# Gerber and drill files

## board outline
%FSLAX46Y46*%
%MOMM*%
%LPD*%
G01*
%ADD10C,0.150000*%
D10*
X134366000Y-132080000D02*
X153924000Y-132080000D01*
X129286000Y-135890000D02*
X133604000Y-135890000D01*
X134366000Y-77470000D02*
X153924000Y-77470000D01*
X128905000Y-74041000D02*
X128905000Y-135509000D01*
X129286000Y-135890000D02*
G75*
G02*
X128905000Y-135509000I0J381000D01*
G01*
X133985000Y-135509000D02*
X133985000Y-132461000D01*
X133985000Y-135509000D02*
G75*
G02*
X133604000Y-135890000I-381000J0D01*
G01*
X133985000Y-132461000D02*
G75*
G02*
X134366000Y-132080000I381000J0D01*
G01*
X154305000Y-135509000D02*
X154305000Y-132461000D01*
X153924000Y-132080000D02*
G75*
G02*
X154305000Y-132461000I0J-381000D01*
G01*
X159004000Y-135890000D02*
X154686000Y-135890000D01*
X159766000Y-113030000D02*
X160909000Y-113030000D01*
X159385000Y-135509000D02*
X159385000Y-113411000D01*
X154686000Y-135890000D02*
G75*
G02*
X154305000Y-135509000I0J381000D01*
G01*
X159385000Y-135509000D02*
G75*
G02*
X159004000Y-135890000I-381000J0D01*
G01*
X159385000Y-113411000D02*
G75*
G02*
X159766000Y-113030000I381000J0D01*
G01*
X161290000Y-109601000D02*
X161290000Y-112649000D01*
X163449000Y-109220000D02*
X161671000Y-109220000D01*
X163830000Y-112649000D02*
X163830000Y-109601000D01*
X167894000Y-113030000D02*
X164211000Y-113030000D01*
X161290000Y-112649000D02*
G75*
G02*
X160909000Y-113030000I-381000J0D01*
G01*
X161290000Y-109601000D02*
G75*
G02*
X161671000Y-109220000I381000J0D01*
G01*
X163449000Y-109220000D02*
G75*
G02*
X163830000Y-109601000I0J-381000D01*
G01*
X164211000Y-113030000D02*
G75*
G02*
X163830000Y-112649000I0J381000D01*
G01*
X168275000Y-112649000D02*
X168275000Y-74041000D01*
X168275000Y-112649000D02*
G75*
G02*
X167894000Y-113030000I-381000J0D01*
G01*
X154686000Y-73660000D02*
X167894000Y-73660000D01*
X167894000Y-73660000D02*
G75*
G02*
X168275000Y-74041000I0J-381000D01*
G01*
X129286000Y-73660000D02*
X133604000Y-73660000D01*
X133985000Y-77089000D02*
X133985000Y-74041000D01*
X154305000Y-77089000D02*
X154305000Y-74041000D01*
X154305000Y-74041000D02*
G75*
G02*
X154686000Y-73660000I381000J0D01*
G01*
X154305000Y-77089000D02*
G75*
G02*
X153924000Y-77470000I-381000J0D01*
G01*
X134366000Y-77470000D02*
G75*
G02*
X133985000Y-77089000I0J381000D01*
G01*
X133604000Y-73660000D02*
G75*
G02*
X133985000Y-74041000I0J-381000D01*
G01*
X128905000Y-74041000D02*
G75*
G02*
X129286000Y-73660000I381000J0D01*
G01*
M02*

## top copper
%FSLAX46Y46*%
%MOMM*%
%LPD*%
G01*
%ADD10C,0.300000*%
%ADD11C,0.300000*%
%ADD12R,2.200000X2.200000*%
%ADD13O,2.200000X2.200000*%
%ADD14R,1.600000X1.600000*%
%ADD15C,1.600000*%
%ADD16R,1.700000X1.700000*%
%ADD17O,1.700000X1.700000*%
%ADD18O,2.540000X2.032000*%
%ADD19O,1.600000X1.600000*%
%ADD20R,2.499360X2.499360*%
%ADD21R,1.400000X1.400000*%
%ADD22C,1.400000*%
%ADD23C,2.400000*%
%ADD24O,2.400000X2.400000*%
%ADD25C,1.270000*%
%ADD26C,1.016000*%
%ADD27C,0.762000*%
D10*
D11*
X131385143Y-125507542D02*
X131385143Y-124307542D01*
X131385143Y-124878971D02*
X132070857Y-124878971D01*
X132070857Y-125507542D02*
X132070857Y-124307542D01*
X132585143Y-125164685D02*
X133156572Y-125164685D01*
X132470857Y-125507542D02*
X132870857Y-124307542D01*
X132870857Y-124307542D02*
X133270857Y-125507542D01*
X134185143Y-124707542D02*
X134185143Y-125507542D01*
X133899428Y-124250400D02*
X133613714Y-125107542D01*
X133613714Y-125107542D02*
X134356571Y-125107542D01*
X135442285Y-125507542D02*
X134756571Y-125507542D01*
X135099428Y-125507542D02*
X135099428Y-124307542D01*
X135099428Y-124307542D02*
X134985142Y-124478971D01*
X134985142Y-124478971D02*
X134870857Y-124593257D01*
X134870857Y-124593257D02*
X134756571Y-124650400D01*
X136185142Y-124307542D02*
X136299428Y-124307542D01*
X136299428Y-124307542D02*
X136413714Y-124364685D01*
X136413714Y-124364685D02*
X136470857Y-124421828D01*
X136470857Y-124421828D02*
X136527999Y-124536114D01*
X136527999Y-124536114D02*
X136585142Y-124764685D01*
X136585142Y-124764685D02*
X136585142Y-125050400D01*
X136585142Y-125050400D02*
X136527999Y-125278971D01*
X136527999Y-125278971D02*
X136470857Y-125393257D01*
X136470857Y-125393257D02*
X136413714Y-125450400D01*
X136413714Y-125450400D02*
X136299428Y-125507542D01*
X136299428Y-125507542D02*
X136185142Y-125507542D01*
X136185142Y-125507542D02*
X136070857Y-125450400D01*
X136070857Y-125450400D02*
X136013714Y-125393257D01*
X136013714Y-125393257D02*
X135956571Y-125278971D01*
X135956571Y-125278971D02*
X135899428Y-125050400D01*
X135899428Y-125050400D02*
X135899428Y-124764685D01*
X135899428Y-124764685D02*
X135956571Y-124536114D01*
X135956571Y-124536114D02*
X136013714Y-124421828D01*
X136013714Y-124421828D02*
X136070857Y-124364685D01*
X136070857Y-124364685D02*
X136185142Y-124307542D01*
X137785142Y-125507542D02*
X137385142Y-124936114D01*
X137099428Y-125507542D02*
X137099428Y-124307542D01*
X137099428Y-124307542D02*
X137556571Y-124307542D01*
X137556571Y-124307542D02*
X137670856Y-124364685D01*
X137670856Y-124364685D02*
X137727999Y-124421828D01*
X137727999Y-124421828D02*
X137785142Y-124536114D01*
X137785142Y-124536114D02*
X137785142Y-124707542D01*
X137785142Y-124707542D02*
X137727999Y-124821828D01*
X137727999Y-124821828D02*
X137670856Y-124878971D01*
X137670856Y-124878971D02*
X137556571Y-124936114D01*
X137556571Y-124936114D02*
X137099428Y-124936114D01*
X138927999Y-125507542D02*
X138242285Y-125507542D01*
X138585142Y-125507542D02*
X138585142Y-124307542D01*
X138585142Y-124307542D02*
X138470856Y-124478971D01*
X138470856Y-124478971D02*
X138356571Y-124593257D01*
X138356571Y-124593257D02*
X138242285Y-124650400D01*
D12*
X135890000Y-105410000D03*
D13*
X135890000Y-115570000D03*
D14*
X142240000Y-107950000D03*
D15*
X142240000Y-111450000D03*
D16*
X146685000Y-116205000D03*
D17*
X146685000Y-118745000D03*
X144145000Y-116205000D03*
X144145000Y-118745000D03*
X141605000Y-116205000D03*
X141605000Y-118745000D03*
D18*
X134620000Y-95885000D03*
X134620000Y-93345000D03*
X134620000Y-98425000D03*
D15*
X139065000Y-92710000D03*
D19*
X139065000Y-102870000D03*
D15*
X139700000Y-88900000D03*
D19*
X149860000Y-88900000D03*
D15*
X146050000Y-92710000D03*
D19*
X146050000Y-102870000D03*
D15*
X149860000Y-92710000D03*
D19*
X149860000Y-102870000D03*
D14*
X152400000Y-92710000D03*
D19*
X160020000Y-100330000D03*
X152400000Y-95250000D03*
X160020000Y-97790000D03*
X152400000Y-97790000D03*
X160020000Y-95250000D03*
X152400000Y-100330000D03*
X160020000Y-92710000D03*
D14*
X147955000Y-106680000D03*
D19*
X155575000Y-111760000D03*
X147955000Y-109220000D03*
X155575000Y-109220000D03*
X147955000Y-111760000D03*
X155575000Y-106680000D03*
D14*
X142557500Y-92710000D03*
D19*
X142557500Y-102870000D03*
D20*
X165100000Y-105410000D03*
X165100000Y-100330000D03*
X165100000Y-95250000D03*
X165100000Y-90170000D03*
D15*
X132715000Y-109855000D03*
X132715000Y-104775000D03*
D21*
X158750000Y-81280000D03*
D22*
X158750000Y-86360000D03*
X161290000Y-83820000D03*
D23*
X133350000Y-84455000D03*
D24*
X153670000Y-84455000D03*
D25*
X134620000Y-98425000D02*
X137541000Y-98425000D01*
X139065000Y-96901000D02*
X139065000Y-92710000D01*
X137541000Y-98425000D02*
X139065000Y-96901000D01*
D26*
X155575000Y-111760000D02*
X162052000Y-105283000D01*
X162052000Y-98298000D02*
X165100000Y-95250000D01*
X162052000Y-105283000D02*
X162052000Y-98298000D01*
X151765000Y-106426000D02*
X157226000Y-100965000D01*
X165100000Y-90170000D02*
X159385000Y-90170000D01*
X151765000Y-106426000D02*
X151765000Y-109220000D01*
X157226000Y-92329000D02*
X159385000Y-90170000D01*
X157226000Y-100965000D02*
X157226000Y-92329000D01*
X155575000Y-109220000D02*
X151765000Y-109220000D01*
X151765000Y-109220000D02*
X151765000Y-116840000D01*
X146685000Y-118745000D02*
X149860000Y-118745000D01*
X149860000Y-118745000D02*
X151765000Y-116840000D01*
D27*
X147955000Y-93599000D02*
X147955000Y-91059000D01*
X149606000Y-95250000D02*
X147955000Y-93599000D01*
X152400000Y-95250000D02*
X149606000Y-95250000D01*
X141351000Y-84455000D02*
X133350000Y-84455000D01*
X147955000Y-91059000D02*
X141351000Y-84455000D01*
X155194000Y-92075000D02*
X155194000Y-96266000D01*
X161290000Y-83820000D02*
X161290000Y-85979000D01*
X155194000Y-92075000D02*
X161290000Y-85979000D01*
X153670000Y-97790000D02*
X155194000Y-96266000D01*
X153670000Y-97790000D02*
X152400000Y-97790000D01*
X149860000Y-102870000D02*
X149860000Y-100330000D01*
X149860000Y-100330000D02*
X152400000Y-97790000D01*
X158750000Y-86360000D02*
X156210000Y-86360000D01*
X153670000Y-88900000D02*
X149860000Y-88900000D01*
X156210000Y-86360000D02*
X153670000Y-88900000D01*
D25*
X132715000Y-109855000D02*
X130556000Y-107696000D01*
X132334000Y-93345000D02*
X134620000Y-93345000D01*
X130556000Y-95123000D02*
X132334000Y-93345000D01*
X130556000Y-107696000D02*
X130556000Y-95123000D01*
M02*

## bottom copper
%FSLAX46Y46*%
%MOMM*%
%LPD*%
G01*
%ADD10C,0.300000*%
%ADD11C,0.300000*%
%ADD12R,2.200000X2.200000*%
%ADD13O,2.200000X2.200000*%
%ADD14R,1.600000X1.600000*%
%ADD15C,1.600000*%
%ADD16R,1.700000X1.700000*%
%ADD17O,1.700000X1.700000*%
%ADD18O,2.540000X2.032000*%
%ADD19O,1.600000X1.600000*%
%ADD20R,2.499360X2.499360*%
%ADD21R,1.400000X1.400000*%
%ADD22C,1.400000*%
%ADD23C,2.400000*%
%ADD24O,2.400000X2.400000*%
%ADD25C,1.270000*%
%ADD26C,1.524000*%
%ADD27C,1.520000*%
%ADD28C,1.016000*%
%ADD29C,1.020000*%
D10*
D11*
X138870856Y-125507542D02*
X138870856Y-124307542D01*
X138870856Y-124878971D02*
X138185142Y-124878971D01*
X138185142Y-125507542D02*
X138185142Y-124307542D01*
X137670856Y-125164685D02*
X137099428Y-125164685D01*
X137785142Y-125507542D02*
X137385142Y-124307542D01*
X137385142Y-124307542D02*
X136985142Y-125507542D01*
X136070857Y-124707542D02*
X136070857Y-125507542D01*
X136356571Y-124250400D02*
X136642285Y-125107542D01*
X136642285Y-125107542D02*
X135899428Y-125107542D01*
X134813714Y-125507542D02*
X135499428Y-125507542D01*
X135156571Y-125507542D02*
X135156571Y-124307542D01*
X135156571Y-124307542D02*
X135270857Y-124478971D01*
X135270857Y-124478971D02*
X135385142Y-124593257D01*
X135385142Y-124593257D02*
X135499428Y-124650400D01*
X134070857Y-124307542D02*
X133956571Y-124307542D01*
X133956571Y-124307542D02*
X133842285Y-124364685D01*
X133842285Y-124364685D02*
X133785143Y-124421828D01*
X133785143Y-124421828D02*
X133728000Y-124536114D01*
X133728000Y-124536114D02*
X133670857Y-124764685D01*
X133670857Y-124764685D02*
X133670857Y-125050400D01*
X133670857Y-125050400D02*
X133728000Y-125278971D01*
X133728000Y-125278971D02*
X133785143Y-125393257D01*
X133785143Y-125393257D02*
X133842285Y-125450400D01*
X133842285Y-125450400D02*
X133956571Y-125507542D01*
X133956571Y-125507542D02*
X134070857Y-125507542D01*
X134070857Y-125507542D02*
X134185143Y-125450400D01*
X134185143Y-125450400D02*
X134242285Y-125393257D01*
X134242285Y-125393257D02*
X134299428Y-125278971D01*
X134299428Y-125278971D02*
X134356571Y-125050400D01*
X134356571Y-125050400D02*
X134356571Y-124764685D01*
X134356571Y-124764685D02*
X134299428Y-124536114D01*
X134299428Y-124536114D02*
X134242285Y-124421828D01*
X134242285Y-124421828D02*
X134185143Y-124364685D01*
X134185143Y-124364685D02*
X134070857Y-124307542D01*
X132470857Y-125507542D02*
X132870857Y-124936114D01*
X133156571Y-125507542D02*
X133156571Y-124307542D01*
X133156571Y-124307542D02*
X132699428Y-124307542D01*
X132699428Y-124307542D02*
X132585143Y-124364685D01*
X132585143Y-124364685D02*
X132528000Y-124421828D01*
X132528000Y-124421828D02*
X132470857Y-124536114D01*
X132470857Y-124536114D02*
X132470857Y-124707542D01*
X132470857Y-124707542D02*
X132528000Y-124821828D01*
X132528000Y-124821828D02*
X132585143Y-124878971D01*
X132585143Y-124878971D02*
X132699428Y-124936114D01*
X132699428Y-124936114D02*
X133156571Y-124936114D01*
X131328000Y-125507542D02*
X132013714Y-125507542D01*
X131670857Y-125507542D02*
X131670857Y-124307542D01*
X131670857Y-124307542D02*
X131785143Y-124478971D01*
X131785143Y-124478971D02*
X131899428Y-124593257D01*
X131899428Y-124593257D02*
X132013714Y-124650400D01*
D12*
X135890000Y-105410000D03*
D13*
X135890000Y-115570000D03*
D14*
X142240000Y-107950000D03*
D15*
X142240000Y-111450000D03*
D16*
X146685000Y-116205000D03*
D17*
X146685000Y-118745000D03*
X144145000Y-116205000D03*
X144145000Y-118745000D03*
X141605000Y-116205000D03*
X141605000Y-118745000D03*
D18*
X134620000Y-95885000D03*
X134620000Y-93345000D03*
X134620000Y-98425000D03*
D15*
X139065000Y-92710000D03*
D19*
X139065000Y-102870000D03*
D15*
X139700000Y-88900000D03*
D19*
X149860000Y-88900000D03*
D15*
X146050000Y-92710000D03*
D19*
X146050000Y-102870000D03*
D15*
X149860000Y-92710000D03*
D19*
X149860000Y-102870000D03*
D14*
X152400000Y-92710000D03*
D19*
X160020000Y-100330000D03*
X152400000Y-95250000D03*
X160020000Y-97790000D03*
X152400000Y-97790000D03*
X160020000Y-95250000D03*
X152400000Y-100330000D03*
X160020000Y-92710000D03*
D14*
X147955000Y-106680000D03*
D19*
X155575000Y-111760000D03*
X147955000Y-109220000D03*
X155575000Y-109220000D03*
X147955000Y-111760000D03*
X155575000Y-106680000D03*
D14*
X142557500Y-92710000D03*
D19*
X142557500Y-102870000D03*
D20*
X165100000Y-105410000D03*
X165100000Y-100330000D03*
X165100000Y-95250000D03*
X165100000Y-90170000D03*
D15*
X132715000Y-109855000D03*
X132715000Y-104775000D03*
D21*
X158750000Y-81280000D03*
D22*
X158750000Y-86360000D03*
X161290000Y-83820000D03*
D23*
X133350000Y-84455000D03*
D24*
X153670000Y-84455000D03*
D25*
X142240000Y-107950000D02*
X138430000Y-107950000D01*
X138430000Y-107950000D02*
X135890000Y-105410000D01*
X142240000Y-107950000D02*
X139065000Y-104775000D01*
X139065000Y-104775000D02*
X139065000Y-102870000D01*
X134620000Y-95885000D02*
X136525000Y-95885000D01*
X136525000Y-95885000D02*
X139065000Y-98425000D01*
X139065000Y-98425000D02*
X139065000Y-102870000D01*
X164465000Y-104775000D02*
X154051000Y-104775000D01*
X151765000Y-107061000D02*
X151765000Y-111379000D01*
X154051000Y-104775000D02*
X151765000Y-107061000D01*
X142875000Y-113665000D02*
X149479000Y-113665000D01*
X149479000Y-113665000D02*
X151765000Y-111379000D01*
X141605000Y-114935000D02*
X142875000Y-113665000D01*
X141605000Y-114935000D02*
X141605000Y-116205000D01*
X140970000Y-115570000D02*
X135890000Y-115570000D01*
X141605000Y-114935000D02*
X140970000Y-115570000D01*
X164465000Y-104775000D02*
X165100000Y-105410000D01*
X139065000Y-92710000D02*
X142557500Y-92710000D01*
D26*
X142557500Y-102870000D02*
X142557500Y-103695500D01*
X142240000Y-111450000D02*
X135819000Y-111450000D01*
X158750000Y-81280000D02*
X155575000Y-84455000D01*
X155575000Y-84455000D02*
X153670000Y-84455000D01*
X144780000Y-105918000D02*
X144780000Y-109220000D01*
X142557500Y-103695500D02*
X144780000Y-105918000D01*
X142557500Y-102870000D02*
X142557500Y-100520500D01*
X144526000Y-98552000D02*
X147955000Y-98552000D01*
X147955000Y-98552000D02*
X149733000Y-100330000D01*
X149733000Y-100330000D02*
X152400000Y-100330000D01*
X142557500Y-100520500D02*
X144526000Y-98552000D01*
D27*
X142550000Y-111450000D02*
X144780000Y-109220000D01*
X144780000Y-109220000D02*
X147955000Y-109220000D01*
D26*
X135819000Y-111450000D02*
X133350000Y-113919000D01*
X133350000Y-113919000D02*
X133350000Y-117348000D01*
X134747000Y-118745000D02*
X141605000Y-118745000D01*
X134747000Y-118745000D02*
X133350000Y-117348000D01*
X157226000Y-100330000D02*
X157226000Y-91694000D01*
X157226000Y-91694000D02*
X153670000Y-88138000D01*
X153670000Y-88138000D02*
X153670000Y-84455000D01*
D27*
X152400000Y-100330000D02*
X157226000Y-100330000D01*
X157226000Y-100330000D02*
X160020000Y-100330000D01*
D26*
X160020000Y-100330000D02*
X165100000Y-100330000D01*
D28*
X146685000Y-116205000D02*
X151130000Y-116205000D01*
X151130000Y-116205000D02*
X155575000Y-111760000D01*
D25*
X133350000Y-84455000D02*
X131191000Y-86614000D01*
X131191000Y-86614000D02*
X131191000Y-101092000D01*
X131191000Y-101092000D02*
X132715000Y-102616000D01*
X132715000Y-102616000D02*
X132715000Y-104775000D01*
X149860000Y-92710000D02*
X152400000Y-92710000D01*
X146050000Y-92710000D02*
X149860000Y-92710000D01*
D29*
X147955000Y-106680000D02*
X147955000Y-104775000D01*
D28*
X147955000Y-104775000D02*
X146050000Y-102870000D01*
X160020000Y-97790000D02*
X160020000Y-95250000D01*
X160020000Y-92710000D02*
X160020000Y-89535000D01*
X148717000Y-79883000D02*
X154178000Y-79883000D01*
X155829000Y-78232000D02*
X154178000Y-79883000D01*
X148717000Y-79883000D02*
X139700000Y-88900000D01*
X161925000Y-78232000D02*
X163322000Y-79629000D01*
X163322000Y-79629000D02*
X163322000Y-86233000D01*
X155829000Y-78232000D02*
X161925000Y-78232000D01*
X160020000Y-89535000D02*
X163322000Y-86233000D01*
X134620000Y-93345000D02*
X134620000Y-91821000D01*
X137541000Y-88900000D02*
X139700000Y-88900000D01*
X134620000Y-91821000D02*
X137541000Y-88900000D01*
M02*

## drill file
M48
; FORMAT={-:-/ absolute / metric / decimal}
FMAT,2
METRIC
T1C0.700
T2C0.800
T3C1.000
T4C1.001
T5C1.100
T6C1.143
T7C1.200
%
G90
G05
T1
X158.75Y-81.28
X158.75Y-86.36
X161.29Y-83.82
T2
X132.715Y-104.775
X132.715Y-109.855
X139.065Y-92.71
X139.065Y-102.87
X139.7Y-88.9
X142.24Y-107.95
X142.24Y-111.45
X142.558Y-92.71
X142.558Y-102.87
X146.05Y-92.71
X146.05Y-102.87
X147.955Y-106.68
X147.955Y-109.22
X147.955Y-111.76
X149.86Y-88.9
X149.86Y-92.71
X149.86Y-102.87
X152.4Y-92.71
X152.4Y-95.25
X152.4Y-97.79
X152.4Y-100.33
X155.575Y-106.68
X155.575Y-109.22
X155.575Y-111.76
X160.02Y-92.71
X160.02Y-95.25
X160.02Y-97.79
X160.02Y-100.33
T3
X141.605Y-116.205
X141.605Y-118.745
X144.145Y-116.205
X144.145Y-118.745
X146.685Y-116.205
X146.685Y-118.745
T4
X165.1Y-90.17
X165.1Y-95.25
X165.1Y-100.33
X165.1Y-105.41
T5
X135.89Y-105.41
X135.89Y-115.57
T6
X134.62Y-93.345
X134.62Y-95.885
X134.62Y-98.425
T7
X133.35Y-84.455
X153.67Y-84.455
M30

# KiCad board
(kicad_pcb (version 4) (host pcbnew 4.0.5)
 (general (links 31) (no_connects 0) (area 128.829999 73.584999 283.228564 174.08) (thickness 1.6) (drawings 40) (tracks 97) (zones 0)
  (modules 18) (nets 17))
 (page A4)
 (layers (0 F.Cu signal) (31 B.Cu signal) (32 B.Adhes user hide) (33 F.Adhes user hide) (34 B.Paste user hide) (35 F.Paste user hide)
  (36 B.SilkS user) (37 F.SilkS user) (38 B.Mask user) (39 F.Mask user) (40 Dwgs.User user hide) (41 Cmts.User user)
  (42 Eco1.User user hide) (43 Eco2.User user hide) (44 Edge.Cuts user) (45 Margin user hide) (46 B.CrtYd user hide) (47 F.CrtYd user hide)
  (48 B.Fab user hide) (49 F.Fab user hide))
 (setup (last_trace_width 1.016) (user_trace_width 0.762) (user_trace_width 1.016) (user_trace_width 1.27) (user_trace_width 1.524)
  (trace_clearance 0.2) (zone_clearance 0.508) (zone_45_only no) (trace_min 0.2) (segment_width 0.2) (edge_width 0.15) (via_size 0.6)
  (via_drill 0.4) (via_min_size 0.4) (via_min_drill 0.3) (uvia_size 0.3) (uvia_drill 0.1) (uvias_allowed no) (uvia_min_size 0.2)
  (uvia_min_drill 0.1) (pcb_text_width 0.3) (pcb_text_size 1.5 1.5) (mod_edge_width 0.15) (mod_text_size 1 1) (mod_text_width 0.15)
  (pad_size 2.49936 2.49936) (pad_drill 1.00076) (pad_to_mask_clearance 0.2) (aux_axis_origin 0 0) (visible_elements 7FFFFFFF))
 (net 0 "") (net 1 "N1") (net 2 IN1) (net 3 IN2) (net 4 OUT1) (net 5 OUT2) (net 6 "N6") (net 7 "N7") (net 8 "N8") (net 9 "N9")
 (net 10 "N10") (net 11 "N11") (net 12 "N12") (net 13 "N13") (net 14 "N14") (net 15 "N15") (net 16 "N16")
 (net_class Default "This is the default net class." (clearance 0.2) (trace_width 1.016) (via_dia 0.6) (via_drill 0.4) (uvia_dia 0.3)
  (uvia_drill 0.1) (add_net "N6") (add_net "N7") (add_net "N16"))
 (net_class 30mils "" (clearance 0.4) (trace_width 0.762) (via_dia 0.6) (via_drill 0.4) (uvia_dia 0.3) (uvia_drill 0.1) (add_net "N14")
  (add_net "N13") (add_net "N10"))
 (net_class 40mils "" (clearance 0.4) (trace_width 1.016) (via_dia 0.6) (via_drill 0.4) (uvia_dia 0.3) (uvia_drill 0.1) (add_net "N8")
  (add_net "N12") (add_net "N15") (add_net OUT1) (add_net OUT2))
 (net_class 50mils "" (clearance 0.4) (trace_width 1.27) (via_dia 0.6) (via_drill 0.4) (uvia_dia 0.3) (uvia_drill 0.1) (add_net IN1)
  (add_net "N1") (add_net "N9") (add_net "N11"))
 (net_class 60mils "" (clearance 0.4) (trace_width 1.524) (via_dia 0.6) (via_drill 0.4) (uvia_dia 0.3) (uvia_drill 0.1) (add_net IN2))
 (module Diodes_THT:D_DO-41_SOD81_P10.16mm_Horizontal (layer F.Cu) (at 135.89 105.41 270)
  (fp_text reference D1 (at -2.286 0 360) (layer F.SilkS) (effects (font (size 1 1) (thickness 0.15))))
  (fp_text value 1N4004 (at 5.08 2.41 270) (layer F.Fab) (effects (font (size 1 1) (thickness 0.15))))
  (pad 1 thru_hole rect (at 0 0 270) (size 2.2 2.2) (drill 1.1) (layers *.Cu *.Mask) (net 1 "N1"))
  (pad 2 thru_hole oval (at 10.16 0 270) (size 2.2 2.2) (drill 1.1) (layers *.Cu *.Mask) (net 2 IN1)))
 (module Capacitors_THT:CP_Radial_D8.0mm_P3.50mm (layer F.Cu) (at 142.24 107.95 270)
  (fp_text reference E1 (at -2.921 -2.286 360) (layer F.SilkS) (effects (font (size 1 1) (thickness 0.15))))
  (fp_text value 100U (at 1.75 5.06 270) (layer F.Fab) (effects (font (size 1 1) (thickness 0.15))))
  (pad 1 thru_hole rect (at 0 0 270) (size 1.6 1.6) (drill 0.8) (layers *.Cu *.Mask) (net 1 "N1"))
  (pad 2 thru_hole circle (at 3.5 0 270) (size 1.6 1.6) (drill 0.8) (layers *.Cu *.Mask) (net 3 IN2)))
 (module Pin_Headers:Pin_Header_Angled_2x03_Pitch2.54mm (layer F.Cu) (at 146.685 116.205 270)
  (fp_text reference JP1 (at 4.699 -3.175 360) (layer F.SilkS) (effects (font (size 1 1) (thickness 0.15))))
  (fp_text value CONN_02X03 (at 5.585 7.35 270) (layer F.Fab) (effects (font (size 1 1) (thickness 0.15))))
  (pad 1 thru_hole rect (at 0 0 270) (size 1.7 1.7) (drill 1) (layers *.Cu *.Mask) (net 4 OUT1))
  (pad 2 thru_hole oval (at 2.54 0 270) (size 1.7 1.7) (drill 1) (layers *.Cu *.Mask) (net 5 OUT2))
  (pad 3 thru_hole oval (at 0 2.54 270) (size 1.7 1.7) (drill 1) (layers *.Cu *.Mask) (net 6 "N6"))
  (pad 4 thru_hole oval (at 2.54 2.54 270) (size 1.7 1.7) (drill 1) (layers *.Cu *.Mask) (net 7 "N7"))
  (pad 5 thru_hole oval (at 0 5.08 270) (size 1.7 1.7) (drill 1) (layers *.Cu *.Mask) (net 2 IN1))
  (pad 6 thru_hole oval (at 2.54 5.08 270) (size 1.7 1.7) (drill 1) (layers *.Cu *.Mask) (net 3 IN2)))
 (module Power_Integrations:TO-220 (layer F.Cu) (at 134.62 95.885 90)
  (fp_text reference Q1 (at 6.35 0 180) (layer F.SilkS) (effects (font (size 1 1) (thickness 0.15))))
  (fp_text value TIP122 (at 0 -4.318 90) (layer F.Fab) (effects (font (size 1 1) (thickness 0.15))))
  (pad 2 thru_hole oval (at 0 0 90) (size 2.032 2.54) (drill 1.143) (layers *.Cu *.Mask) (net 1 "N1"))
  (pad 3 thru_hole oval (at 2.54 0 90) (size 2.032 2.54) (drill 1.143) (layers *.Cu *.Mask) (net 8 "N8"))
  (pad 1 thru_hole oval (at -2.54 0 90) (size 2.032 2.54) (drill 1.143) (layers *.Cu *.Mask) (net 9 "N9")))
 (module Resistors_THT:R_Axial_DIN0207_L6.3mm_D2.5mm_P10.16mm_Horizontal (layer F.Cu) (at 139.065 92.71 270)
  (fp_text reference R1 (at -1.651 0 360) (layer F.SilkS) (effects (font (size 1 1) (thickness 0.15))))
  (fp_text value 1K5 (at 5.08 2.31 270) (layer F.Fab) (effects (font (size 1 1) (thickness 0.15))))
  (pad 1 thru_hole circle (at 0 0 270) (size 1.6 1.6) (drill 0.8) (layers *.Cu *.Mask) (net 9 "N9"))
  (pad 2 thru_hole oval (at 10.16 0 270) (size 1.6 1.6) (drill 0.8) (layers *.Cu *.Mask) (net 1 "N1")))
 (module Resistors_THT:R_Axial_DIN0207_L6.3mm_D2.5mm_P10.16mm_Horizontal (layer F.Cu) (at 139.7 88.9)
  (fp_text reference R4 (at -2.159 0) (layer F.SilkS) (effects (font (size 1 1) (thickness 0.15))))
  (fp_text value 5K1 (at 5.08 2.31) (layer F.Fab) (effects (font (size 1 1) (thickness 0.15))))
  (pad 1 thru_hole circle (at 0 0) (size 1.6 1.6) (drill 0.8) (layers *.Cu *.Mask) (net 8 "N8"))
  (pad 2 thru_hole oval (at 10.16 0) (size 1.6 1.6) (drill 0.8) (layers *.Cu *.Mask) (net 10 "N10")))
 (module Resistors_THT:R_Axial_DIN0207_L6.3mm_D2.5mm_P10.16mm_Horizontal (layer F.Cu) (at 146.05 92.71 270)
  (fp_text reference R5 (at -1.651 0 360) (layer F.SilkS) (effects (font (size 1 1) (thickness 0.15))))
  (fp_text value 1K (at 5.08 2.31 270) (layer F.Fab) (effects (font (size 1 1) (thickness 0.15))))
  (pad 1 thru_hole circle (at 0 0 270) (size 1.6 1.6) (drill 0.8) (layers *.Cu *.Mask) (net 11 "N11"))
  (pad 2 thru_hole oval (at 10.16 0 270) (size 1.6 1.6) (drill 0.8) (layers *.Cu *.Mask) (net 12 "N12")))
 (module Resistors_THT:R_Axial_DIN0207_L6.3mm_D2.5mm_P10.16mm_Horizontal (layer F.Cu) (at 149.86 92.71 270)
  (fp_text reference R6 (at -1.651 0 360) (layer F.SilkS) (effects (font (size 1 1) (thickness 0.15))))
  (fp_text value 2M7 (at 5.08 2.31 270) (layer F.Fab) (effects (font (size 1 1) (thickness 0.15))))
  (pad 1 thru_hole circle (at 0 0 270) (size 1.6 1.6) (drill 0.8) (layers *.Cu *.Mask) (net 11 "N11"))
  (pad 2 thru_hole oval (at 10.16 0 270) (size 1.6 1.6) (drill 0.8) (layers *.Cu *.Mask) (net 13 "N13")))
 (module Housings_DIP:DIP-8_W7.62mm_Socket (layer F.Cu) (at 152.4 92.71)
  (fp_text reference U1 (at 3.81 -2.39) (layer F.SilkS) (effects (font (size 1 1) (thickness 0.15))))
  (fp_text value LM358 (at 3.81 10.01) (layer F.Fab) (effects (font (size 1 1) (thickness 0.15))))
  (pad 1 thru_hole rect (at 0 0) (size 1.6 1.6) (drill 0.8) (layers *.Cu *.Mask) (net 11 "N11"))
  (pad 5 thru_hole oval (at 7.62 7.62) (size 1.6 1.6) (drill 0.8) (layers *.Cu *.Mask) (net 3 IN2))
  (pad 2 thru_hole oval (at 0 2.54) (size 1.6 1.6) (drill 0.8) (layers *.Cu *.Mask) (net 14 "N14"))
  (pad 6 thru_hole oval (at 7.62 5.08) (size 1.6 1.6) (drill 0.8) (layers *.Cu *.Mask) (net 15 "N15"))
  (pad 3 thru_hole oval (at 0 5.08) (size 1.6 1.6) (drill 0.8) (layers *.Cu *.Mask) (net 13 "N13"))
  (pad 7 thru_hole oval (at 7.62 2.54) (size 1.6 1.6) (drill 0.8) (layers *.Cu *.Mask) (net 15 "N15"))
  (pad 4 thru_hole oval (at 0 7.62) (size 1.6 1.6) (drill 0.8) (layers *.Cu *.Mask) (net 3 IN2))
  (pad 8 thru_hole oval (at 7.62 0) (size 1.6 1.6) (drill 0.8) (layers *.Cu *.Mask) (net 8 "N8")))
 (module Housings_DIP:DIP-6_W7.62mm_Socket (layer F.Cu) (at 147.955 106.68)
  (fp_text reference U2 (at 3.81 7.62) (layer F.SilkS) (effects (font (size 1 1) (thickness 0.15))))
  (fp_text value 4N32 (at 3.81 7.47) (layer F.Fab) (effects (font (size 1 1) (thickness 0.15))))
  (pad 1 thru_hole rect (at 0 0) (size 1.6 1.6) (drill 0.8) (layers *.Cu *.Mask) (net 12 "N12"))
  (pad 4 thru_hole oval (at 7.62 5.08) (size 1.6 1.6) (drill 0.8) (layers *.Cu *.Mask) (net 4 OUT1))
  (pad 2 thru_hole oval (at 0 2.54) (size 1.6 1.6) (drill 0.8) (layers *.Cu *.Mask) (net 3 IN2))
  (pad 5 thru_hole oval (at 7.62 2.54) (size 1.6 1.6) (drill 0.8) (layers *.Cu *.Mask) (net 5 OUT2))
  (pad 3 thru_hole oval (at 0 5.08) (size 1.6 1.6) (drill 0.8) (layers *.Cu *.Mask))
  (pad 6 thru_hole oval (at 7.62 0) (size 1.6 1.6) (drill 0.8) (layers *.Cu *.Mask) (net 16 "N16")))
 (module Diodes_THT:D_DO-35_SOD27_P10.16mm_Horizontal (layer F.Cu) (at 142.5575 92.71 270)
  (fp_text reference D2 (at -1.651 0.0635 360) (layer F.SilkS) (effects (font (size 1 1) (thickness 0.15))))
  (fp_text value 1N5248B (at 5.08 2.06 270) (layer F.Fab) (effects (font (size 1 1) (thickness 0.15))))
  (pad 1 thru_hole rect (at 0 0 270) (size 1.6 1.6) (drill 0.8) (layers *.Cu *.Mask) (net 9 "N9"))
  (pad 2 thru_hole oval (at 10.16 0 270) (size 1.6 1.6) (drill 0.8) (layers *.Cu *.Mask) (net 3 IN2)))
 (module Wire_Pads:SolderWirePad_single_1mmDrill (layer F.Cu) (at 165.1 105.41)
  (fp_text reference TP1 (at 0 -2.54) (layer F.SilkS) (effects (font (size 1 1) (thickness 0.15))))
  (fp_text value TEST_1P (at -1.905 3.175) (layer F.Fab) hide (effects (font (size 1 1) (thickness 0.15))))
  (pad 1 thru_hole rect (at 0 0) (size 2.49936 2.49936) (drill 1.00076) (layers *.Cu *.Mask) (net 2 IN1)))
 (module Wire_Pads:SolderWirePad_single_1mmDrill (layer F.Cu) (at 165.1 100.33)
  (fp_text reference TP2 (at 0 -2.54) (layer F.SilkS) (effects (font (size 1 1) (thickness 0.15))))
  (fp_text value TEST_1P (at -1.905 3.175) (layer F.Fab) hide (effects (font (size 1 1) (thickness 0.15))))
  (pad 1 thru_hole rect (at 0 0) (size 2.49936 2.49936) (drill 1.00076) (layers *.Cu *.Mask) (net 3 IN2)))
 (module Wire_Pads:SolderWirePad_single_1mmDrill (layer F.Cu) (at 165.1 95.25)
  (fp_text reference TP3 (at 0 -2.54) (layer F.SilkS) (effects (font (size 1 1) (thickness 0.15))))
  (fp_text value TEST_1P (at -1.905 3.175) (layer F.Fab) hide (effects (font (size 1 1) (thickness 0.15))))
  (pad 1 thru_hole rect (at 0 0) (size 2.49936 2.49936) (drill 1.00076) (layers *.Cu *.Mask) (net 4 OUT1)))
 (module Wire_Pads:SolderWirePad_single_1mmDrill (layer F.Cu) (at 165.1 90.17)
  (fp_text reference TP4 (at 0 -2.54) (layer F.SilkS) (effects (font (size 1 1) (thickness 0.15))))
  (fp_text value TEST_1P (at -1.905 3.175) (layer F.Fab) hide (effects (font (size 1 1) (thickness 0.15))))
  (pad 1 thru_hole rect (at 0 0) (size 2.49936 2.49936) (drill 1.00076) (layers *.Cu *.Mask) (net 5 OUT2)))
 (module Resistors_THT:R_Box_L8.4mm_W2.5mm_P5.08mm (layer F.Cu) (at 132.715 109.855 90)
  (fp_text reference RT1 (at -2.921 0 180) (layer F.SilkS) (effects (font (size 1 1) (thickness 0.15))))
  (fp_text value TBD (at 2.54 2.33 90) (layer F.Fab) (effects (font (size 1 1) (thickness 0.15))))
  (pad 1 thru_hole circle (at 0 0 90) (size 1.6 1.6) (drill 0.8) (layers *.Cu *.Mask) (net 8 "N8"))
  (pad 2 thru_hole circle (at 5.08 0 90) (size 1.6 1.6) (drill 0.8) (layers *.Cu *.Mask) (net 14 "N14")))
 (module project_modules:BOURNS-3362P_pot (layer F.Cu) (at 158.75 83.82 270)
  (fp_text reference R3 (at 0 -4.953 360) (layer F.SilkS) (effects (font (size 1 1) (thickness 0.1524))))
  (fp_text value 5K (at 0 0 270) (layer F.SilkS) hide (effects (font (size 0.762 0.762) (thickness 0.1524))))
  (pad 1 thru_hole rect (at -2.54 0 270) (size 1.4 1.4) (drill 0.7) (layers *.Cu *.Mask F.SilkS) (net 3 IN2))
  (pad 3 thru_hole circle (at 2.54 0 270) (size 1.4 1.4) (drill 0.7) (layers *.Cu *.Mask F.SilkS) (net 10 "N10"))
  (pad 2 thru_hole circle (at 0 -2.54 270) (size 1.4 1.4) (drill 0.7) (layers *.Cu *.Mask F.SilkS) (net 13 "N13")))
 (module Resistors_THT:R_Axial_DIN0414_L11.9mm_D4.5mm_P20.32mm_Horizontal (layer F.Cu) (at 133.35 84.455)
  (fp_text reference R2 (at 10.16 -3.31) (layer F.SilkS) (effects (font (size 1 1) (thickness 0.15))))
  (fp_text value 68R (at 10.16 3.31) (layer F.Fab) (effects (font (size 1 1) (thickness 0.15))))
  (pad 1 thru_hole circle (at 0 0) (size 2.4 2.4) (drill 1.2) (layers *.Cu *.Mask) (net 14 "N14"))
  (pad 2 thru_hole oval (at 20.32 0) (size 2.4 2.4) (drill 1.2) (layers *.Cu *.Mask) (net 3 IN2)))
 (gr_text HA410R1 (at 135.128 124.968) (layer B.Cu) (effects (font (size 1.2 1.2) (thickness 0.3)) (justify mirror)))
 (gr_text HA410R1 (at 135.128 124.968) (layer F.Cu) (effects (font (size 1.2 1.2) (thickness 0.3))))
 (gr_line (start 134.366 132.08) (end 153.924 132.08) (angle 90) (layer Edge.Cuts) (width 0.15))
 (gr_line (start 129.286 135.89) (end 133.604 135.89) (angle 90) (layer Edge.Cuts) (width 0.15))
 (gr_line (start 134.366 77.47) (end 153.924 77.47) (angle 90) (layer Edge.Cuts) (width 0.15))
 (gr_line (start 128.905 74.041) (end 128.905 135.509) (angle 90) (layer Edge.Cuts) (width 0.15))
 (gr_arc (start 129.286 135.509) (end 129.286 135.89) (angle 90) (layer Edge.Cuts) (width 0.15))
 (gr_line (start 133.985 135.509) (end 133.985 132.461) (angle 90) (layer Edge.Cuts) (width 0.15))
 (gr_arc (start 133.604 135.509) (end 133.604 135.89) (angle -90) (layer Edge.Cuts) (width 0.15))
 (gr_arc (start 134.366 132.461) (end 134.366 132.08) (angle -90) (layer Edge.Cuts) (width 0.15))
 (gr_line (start 154.305 135.509) (end 154.305 132.461) (angle 90) (layer Edge.Cuts) (width 0.15))
 (gr_arc (start 153.924 132.461) (end 153.924 132.08) (angle 90) (layer Edge.Cuts) (width 0.15))
 (gr_line (start 159.004 135.89) (end 154.686 135.89) (angle 90) (layer Edge.Cuts) (width 0.15))
 (gr_line (start 159.766 113.03) (end 160.909 113.03) (angle 90) (layer Edge.Cuts) (width 0.15))
 (gr_line (start 159.385 135.509) (end 159.385 113.411) (angle 90) (layer Edge.Cuts) (width 0.15))
 (gr_arc (start 154.686 135.509) (end 154.686 135.89) (angle 90) (layer Edge.Cuts) (width 0.15))
 (gr_arc (start 159.004 135.509) (end 159.004 135.89) (angle -90) (layer Edge.Cuts) (width 0.15))
 (gr_arc (start 159.766 113.411) (end 159.766 113.03) (angle -90) (layer Edge.Cuts) (width 0.15))
 (gr_line (start 161.29 109.601) (end 161.29 112.649) (angle 90) (layer Edge.Cuts) (width 0.15))
 (gr_line (start 163.449 109.22) (end 161.671 109.22) (angle 90) (layer Edge.Cuts) (width 0.15))
 (gr_line (start 163.83 112.649) (end 163.83 109.601) (angle 90) (layer Edge.Cuts) (width 0.15))
 (gr_line (start 167.894 113.03) (end 164.211 113.03) (angle 90) (layer Edge.Cuts) (width 0.15))
 (gr_arc (start 160.909 112.649) (end 160.909 113.03) (angle -90) (layer Edge.Cuts) (width 0.15))
 (gr_arc (start 161.671 109.601) (end 161.671 109.22) (angle -90) (layer Edge.Cuts) (width 0.15))
 (gr_arc (start 163.449 109.601) (end 163.449 109.22) (angle 90) (layer Edge.Cuts) (width 0.15))
 (gr_arc (start 164.211 112.649) (end 164.211 113.03) (angle 90) (layer Edge.Cuts) (width 0.15))
 (gr_line (start 168.275 112.649) (end 168.275 74.041) (angle 90) (layer Edge.Cuts) (width 0.15))
 (gr_arc (start 167.894 112.649) (end 167.894 113.03) (angle -90) (layer Edge.Cuts) (width 0.15))
 (gr_line (start 154.686 73.66) (end 167.894 73.66) (angle 90) (layer Edge.Cuts) (width 0.15))
 (gr_arc (start 167.894 74.041) (end 167.894 73.66) (angle 90) (layer Edge.Cuts) (width 0.15))
 (gr_line (start 129.286 73.66) (end 133.604 73.66) (angle 90) (layer Edge.Cuts) (width 0.15))
 (gr_line (start 133.985 77.089) (end 133.985 74.041) (angle 90) (layer Edge.Cuts) (width 0.15))
 (gr_line (start 154.305 77.089) (end 154.305 74.041) (angle 90) (layer Edge.Cuts) (width 0.15))
 (gr_arc (start 154.686 74.041) (end 154.686 73.66) (angle -90) (layer Edge.Cuts) (width 0.15))
 (gr_arc (start 153.924 77.089) (end 153.924 77.47) (angle -90) (layer Edge.Cuts) (width 0.15))
 (gr_arc (start 134.366 77.089) (end 134.366 77.47) (angle 90) (layer Edge.Cuts) (width 0.15))
 (gr_arc (start 133.604 74.041) (end 133.604 73.66) (angle 90) (layer Edge.Cuts) (width 0.15))
 (gr_arc (start 129.286 74.041) (end 129.286 73.66) (angle -90) (layer Edge.Cuts) (width 0.15))
 (segment (start 142.24 107.95) (end 138.43 107.95) (width 1.27) (layer B.Cu) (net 1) (status 10))
 (segment (start 138.43 107.95) (end 135.89 105.41) (width 1.27) (layer B.Cu) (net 1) (status 20))
 (segment (start 142.24 107.95) (end 139.065 104.775) (width 1.27) (layer B.Cu) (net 1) (status 10))
 (segment (start 139.065 104.775) (end 139.065 102.87) (width 1.27) (layer B.Cu) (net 1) (status 20))
 (segment (start 134.62 95.885) (end 136.525 95.885) (width 1.27) (layer B.Cu) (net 1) (status 10))
 (segment (start 136.525 95.885) (end 139.065 98.425) (width 1.27) (layer B.Cu) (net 1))
 (segment (start 139.065 98.425) (end 139.065 102.87) (width 1.27) (layer B.Cu) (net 1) (status 20))
 (segment (start 164.465 104.775) (end 154.051 104.775) (width 1.27) (layer B.Cu) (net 2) (status 10))
 (segment (start 151.765 107.061) (end 151.765 111.379) (width 1.27) (layer B.Cu) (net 2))
 (segment (start 154.051 104.775) (end 151.765 107.061) (width 1.27) (layer B.Cu) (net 2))
 (segment (start 142.875 113.665) (end 149.479 113.665) (width 1.27) (layer B.Cu) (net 2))
 (segment (start 149.479 113.665) (end 151.765 111.379) (width 1.27) (layer B.Cu) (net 2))
 (segment (start 141.605 114.935) (end 142.875 113.665) (width 1.27) (layer B.Cu) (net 2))
 (segment (start 141.605 114.935) (end 141.605 116.205) (width 1.27) (layer B.Cu) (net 2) (status 20))
 (segment (start 140.97 115.57) (end 135.89 115.57) (width 1.27) (layer B.Cu) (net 2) (status 20))
 (segment (start 141.605 114.935) (end 140.97 115.57) (width 1.27) (layer B.Cu) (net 2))
 (segment (start 164.465 104.775) (end 165.1 105.41) (width 1.27) (layer B.Cu) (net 2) (status 30))
 (segment (start 134.62 98.425) (end 137.541 98.425) (width 1.27) (layer F.Cu) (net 9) (status 10))
 (segment (start 139.065 96.901) (end 139.065 92.71) (width 1.27) (layer F.Cu) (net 9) (status 20))
 (segment (start 137.541 98.425) (end 139.065 96.901) (width 1.27) (layer F.Cu) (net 9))
 (segment (start 139.065 92.71) (end 142.5575 92.71) (width 1.27) (layer B.Cu) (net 9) (status 30))
 (segment (start 142.5575 102.87) (end 142.5575 103.6955) (width 1.524) (layer B.Cu) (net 3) (status 10))
 (segment (start 142.24 111.45) (end 135.819 111.45) (width 1.524) (layer B.Cu) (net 3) (status 10))
 (segment (start 158.75 81.28) (end 155.575 84.455) (width 1.524) (layer B.Cu) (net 3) (status 10))
 (segment (start 155.575 84.455) (end 153.67 84.455) (width 1.524) (layer B.Cu) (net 3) (status 20))
 (segment (start 144.78 105.918) (end 144.78 109.22) (width 1.524) (layer B.Cu) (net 3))
 (segment (start 142.5575 103.6955) (end 144.78 105.918) (width 1.524) (layer B.Cu) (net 3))
 (segment (start 142.5575 102.87) (end 142.5575 100.5205) (width 1.524) (layer B.Cu) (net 3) (status 10))
 (segment (start 144.526 98.552) (end 147.955 98.552) (width 1.524) (layer B.Cu) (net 3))
 (segment (start 147.955 98.552) (end 149.733 100.33) (width 1.524) (layer B.Cu) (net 3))
 (segment (start 149.733 100.33) (end 152.4 100.33) (width 1.524) (layer B.Cu) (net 3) (status 20))
 (segment (start 142.5575 100.5205) (end 144.526 98.552) (width 1.524) (layer B.Cu) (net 3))
 (segment (start 142.55 111.45) (end 144.78 109.22) (width 1.52) (layer B.Cu) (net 3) (status 10))
 (segment (start 144.78 109.22) (end 147.955 109.22) (width 1.52) (layer B.Cu) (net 3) (status 20))
 (segment (start 135.819 111.45) (end 133.35 113.919) (width 1.524) (layer B.Cu) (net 3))
 (segment (start 133.35 113.919) (end 133.35 117.348) (width 1.524) (layer B.Cu) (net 3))
 (segment (start 134.747 118.745) (end 141.605 118.745) (width 1.524) (layer B.Cu) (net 3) (status 20))
 (segment (start 134.747 118.745) (end 133.35 117.348) (width 1.524) (layer B.Cu) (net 3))
 (segment (start 157.226 100.33) (end 157.226 91.694) (width 1.524) (layer B.Cu) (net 3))
 (segment (start 157.226 91.694) (end 153.67 88.138) (width 1.524) (layer B.Cu) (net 3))
 (segment (start 153.67 88.138) (end 153.67 84.455) (width 1.524) (layer B.Cu) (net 3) (status 20))
 (segment (start 152.4 100.33) (end 157.226 100.33) (width 1.52) (layer B.Cu) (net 3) (status 10))
 (segment (start 157.226 100.33) (end 160.02 100.33) (width 1.52) (layer B.Cu) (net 3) (status 20))
 (segment (start 160.02 100.33) (end 165.1 100.33) (width 1.524) (layer B.Cu) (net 3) (status 30))
 (segment (start 155.575 111.76) (end 162.052 105.283) (width 1.016) (layer F.Cu) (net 4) (status 10))
 (segment (start 162.052 98.298) (end 165.1 95.25) (width 1.016) (layer F.Cu) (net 4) (status 20))
 (segment (start 162.052 105.283) (end 162.052 98.298) (width 1.016) (layer F.Cu) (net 4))
 (segment (start 146.685 116.205) (end 151.13 116.205) (width 1.016) (layer B.Cu) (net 4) (status 10))
 (segment (start 151.13 116.205) (end 155.575 111.76) (width 1.016) (layer B.Cu) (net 4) (status 20))
 (segment (start 151.765 106.426) (end 157.226 100.965) (width 1.016) (layer F.Cu) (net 5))
 (segment (start 165.1 90.17) (end 159.385 90.17) (width 1.016) (layer F.Cu) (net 5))
 (segment (start 151.765 106.426) (end 151.765 109.22) (width 1.016) (layer F.Cu) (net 5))
 (segment (start 157.226 92.329) (end 159.385 90.17) (width 1.016) (layer F.Cu) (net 5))
 (segment (start 157.226 100.965) (end 157.226 92.329) (width 1.016) (layer F.Cu) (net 5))
 (segment (start 155.575 109.22) (end 151.765 109.22) (width 1.016) (layer F.Cu) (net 5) (status 10))
 (segment (start 151.765 109.22) (end 151.765 116.84) (width 1.016) (layer F.Cu) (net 5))
 (segment (start 146.685 118.745) (end 149.86 118.745) (width 1.016) (layer F.Cu) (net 5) (status 10))
 (segment (start 149.86 118.745) (end 151.765 116.84) (width 1.016) (layer F.Cu) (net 5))
 (segment (start 147.955 93.599) (end 147.955 91.059) (width 0.762) (layer F.Cu) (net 14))
 (segment (start 149.606 95.25) (end 147.955 93.599) (width 0.762) (layer F.Cu) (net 14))
 (segment (start 152.4 95.25) (end 149.606 95.25) (width 0.762) (layer F.Cu) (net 14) (status 10))
 (segment (start 141.351 84.455) (end 133.35 84.455) (width 0.762) (layer F.Cu) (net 14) (status 20))
 (segment (start 147.955 91.059) (end 141.351 84.455) (width 0.762) (layer F.Cu) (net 14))
 (segment (start 133.35 84.455) (end 131.191 86.614) (width 1.27) (layer B.Cu) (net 14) (status 10))
 (segment (start 131.191 86.614) (end 131.191 101.092) (width 1.27) (layer B.Cu) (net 14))
 (segment (start 131.191 101.092) (end 132.715 102.616) (width 1.27) (layer B.Cu) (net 14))
 (segment (start 132.715 102.616) (end 132.715 104.775) (width 1.27) (layer B.Cu) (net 14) (status 20))
 (segment (start 155.194 92.075) (end 155.194 96.266) (width 0.762) (layer F.Cu) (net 13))
 (segment (start 161.29 83.82) (end 161.29 85.979) (width 0.762) (layer F.Cu) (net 13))
 (segment (start 155.194 92.075) (end 161.29 85.979) (width 0.762) (layer F.Cu) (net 13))
 (segment (start 153.67 97.79) (end 155.194 96.266) (width 0.762) (layer F.Cu) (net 13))
 (segment (start 153.67 97.79) (end 152.4 97.79) (width 0.762) (layer F.Cu) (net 13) (status 10))
 (segment (start 149.86 102.87) (end 149.86 100.33) (width 0.762) (layer F.Cu) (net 13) (status 10))
 (segment (start 149.86 100.33) (end 152.4 97.79) (width 0.762) (layer F.Cu) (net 13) (status 20))
 (segment (start 149.86 92.71) (end 152.4 92.71) (width 1.27) (layer B.Cu) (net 11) (status 30))
 (segment (start 146.05 92.71) (end 149.86 92.71) (width 1.27) (layer B.Cu) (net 11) (status 30))
 (segment (start 147.955 106.68) (end 147.955 104.775) (width 1.02) (layer B.Cu) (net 12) (status 10))
 (segment (start 147.955 104.775) (end 146.05 102.87) (width 1.016) (layer B.Cu) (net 12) (status 20))
 (segment (start 160.02 97.79) (end 160.02 95.25) (width 1.016) (layer B.Cu) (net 15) (status 30))
 (segment (start 158.75 86.36) (end 156.21 86.36) (width 0.762) (layer F.Cu) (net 10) (status 10))
 (segment (start 153.67 88.9) (end 149.86 88.9) (width 0.762) (layer F.Cu) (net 10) (status 20))
 (segment (start 156.21 86.36) (end 153.67 88.9) (width 0.762) (layer F.Cu) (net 10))
 (segment (start 160.02 92.71) (end 160.02 89.535) (width 1.016) (layer B.Cu) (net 8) (status 10))
 (segment (start 148.717 79.883) (end 154.178 79.883) (width 1.016) (layer B.Cu) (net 8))
 (segment (start 155.829 78.232) (end 154.178 79.883) (width 1.016) (layer B.Cu) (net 8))
 (segment (start 148.717 79.883) (end 139.7 88.9) (width 1.016) (layer B.Cu) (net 8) (status 20))
 (segment (start 161.925 78.232) (end 163.322 79.629) (width 1.016) (layer B.Cu) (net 8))
 (segment (start 163.322 79.629) (end 163.322 86.233) (width 1.016) (layer B.Cu) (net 8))
 (segment (start 155.829 78.232) (end 161.925 78.232) (width 1.016) (layer B.Cu) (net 8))
 (segment (start 160.02 89.535) (end 163.322 86.233) (width 1.016) (layer B.Cu) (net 8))
 (segment (start 134.62 93.345) (end 134.62 91.821) (width 1.016) (layer B.Cu) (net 8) (status 10))
 (segment (start 137.541 88.9) (end 139.7 88.9) (width 1.016) (layer B.Cu) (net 8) (status 20))
 (segment (start 134.62 91.821) (end 137.541 88.9) (width 1.016) (layer B.Cu) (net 8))
 (segment (start 132.715 109.855) (end 130.556 107.696) (width 1.27) (layer F.Cu) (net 8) (status 10))
 (segment (start 132.334 93.345) (end 134.62 93.345) (width 1.27) (layer F.Cu) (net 8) (status 20))
 (segment (start 130.556 95.123) (end 132.334 93.345) (width 1.27) (layer F.Cu) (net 8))
 (segment (start 130.556 107.696) (end 130.556 95.123) (width 1.27) (layer F.Cu) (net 8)))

